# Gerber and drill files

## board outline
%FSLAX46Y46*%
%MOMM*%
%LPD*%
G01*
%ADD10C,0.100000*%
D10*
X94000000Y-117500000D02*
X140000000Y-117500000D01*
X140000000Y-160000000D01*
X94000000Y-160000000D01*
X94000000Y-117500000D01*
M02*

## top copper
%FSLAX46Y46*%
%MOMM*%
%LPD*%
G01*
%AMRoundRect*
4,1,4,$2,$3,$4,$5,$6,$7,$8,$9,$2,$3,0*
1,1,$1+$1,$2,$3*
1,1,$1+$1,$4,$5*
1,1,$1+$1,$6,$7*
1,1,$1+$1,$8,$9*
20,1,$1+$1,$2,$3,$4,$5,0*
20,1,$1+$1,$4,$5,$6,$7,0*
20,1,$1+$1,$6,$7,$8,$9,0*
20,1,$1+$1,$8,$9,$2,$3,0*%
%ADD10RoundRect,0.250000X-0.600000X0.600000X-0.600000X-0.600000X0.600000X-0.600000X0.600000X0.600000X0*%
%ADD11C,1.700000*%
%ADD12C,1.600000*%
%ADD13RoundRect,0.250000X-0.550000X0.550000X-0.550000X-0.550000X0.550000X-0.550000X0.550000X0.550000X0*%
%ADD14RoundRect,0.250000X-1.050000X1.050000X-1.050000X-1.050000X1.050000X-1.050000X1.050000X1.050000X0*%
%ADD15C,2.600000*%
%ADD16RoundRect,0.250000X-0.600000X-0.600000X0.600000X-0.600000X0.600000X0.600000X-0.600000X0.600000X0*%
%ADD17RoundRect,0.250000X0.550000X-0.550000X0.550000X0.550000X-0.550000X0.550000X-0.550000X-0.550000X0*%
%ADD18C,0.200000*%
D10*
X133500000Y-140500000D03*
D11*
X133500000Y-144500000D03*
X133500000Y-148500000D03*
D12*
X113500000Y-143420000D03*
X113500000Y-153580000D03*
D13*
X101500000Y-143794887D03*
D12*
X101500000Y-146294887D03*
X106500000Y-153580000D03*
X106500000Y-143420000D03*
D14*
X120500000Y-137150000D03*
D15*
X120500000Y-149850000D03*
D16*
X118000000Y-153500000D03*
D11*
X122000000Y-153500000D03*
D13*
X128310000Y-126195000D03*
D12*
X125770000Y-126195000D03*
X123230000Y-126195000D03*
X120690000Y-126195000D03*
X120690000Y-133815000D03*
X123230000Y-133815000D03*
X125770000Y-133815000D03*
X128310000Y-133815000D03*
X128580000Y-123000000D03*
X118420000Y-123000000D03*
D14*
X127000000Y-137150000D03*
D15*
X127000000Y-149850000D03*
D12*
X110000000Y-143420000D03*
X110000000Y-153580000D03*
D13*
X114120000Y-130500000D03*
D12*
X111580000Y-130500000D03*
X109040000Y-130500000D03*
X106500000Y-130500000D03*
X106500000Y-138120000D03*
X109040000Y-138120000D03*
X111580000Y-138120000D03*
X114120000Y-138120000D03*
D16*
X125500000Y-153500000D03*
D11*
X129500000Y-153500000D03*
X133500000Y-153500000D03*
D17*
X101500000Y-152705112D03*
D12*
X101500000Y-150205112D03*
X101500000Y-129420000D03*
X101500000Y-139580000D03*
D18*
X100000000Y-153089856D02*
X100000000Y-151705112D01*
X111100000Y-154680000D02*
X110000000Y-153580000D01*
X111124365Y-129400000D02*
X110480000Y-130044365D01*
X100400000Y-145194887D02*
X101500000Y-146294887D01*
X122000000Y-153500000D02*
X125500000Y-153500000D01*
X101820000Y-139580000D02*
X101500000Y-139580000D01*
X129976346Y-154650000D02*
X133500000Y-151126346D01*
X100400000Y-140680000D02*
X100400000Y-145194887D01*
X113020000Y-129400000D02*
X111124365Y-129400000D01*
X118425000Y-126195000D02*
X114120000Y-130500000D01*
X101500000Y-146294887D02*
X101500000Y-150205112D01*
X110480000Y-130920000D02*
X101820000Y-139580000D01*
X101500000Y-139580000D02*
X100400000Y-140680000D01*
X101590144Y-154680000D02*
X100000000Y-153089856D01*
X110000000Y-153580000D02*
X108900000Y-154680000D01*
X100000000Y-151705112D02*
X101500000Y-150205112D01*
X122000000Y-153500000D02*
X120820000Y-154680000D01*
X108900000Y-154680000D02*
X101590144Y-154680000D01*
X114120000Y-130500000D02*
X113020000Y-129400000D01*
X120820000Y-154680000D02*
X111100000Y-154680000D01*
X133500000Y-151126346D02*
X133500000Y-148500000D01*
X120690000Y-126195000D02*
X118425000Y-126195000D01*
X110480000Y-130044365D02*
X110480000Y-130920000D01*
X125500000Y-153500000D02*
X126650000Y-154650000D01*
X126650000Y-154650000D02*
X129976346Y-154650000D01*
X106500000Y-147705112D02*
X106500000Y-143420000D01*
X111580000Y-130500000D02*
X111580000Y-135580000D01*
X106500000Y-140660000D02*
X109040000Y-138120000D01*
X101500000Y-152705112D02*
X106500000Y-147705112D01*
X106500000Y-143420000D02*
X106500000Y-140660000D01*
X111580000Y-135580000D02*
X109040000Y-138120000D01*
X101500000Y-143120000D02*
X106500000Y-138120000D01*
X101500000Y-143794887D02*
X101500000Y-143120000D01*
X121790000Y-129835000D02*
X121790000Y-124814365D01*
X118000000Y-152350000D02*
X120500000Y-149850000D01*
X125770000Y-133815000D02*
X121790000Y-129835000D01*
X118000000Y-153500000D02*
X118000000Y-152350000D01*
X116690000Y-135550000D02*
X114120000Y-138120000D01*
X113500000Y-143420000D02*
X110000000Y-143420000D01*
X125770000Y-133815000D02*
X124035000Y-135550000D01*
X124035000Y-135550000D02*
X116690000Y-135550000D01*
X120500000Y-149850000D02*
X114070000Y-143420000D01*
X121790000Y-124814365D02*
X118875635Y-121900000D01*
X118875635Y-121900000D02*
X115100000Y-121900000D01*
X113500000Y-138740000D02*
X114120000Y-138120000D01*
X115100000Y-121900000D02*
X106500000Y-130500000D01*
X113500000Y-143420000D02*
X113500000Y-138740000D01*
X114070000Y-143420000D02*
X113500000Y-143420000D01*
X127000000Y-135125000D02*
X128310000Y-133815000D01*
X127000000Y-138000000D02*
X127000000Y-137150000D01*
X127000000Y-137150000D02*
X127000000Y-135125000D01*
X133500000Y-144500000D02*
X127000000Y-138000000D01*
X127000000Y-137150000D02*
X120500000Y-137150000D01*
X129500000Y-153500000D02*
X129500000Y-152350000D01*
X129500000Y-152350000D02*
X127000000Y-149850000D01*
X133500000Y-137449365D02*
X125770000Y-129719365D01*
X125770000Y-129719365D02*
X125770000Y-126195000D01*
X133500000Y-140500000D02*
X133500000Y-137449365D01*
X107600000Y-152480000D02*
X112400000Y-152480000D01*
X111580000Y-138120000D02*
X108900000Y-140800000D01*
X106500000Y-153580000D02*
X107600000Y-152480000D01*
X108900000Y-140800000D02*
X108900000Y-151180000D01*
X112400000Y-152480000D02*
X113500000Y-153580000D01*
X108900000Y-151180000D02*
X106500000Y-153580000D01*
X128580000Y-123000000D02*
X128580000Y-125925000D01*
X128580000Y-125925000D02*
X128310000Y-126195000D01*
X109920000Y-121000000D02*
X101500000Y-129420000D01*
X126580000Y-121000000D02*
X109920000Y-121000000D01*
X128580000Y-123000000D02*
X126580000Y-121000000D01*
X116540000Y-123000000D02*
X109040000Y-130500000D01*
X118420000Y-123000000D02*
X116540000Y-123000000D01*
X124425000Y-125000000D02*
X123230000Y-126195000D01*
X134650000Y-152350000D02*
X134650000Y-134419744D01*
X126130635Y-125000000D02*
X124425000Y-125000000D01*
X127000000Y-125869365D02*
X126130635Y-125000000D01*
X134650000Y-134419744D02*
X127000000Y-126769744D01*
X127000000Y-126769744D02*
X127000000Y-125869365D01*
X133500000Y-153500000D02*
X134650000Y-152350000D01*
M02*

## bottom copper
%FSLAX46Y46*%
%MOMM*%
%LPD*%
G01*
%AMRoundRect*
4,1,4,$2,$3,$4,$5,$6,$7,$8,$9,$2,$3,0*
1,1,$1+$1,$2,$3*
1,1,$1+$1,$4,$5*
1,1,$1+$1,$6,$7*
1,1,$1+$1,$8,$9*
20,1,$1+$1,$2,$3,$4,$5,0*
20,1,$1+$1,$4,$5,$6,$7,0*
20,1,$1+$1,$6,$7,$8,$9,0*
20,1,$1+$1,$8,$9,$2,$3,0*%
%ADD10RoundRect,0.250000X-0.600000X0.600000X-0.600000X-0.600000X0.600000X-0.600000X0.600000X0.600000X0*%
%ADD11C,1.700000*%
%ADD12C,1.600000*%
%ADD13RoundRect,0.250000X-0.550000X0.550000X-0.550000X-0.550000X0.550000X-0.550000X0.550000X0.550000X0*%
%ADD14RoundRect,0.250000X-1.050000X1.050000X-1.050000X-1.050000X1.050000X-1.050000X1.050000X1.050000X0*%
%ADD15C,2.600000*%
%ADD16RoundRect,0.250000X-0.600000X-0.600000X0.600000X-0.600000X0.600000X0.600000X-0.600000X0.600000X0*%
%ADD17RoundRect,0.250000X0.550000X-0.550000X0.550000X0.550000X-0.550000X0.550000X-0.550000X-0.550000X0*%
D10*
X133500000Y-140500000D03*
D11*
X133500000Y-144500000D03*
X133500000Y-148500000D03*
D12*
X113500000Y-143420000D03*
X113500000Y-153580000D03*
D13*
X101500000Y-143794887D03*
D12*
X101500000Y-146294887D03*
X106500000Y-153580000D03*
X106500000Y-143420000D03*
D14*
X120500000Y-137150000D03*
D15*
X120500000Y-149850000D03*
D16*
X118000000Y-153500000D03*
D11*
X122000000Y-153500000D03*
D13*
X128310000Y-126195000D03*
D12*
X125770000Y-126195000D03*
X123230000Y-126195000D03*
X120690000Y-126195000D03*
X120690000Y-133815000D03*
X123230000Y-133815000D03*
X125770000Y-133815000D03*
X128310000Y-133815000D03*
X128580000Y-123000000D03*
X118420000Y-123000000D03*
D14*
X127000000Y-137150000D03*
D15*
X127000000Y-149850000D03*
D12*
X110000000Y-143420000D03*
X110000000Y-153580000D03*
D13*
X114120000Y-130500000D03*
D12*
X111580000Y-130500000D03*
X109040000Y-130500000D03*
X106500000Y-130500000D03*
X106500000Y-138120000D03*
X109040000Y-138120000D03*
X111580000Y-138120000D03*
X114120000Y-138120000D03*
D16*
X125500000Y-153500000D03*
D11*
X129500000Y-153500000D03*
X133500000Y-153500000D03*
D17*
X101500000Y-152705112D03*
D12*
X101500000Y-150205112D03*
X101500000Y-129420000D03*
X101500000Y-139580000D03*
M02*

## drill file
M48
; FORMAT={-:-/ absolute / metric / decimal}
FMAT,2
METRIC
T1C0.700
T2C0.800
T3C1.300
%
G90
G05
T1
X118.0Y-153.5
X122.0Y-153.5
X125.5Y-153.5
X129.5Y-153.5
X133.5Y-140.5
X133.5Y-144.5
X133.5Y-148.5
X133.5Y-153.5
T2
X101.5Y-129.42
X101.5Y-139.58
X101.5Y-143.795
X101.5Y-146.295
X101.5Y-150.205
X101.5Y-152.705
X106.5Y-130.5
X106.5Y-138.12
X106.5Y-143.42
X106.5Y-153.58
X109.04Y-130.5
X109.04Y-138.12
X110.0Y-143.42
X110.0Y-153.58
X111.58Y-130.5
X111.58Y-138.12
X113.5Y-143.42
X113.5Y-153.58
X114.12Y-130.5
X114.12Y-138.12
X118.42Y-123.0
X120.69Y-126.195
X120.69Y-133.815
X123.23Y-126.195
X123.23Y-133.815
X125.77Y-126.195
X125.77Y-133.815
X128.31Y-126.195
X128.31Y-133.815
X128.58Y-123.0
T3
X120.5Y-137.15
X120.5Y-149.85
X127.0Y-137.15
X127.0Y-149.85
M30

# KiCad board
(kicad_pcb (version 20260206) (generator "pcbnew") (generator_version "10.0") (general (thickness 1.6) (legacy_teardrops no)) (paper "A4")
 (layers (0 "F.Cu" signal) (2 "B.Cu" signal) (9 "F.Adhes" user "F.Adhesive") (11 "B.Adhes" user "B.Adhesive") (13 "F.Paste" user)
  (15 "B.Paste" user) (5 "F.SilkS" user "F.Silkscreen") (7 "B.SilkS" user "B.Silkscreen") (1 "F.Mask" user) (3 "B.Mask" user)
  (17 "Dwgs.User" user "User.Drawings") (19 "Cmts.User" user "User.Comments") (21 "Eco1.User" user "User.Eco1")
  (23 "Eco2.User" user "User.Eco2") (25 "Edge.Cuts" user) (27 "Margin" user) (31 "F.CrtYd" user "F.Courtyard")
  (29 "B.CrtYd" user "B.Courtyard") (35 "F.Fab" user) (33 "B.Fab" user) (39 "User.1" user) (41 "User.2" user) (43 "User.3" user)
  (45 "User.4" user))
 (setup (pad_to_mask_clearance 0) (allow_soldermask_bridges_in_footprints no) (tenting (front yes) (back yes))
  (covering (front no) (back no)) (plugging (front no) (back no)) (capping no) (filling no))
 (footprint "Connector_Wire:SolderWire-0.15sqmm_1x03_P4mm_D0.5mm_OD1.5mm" (layer "F.Cu") (at 133.5 140.5 -90)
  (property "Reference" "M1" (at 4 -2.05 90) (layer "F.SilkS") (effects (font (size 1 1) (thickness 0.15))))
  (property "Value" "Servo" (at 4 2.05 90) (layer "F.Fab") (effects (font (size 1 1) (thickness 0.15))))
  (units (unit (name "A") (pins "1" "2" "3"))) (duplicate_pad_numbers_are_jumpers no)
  (pad "1" thru_hole roundrect (at 0 0 270) (size 1.7 1.7) (drill 0.7) (layers "*.Cu" "*.Mask") (remove_unused_layers no)
   (roundrect_rratio 0.147059) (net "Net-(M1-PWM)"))
  (pad "2" thru_hole circle (at 4 0 270) (size 1.7 1.7) (drill 0.7) (layers "*.Cu" "*.Mask") (remove_unused_layers no) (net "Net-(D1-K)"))
  (pad "3" thru_hole circle (at 8 0 270) (size 1.7 1.7) (drill 0.7) (layers "*.Cu" "*.Mask") (remove_unused_layers no) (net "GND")))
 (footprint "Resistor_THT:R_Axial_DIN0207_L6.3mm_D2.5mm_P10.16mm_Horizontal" (layer "F.Cu") (at 113.5 143.42 -90)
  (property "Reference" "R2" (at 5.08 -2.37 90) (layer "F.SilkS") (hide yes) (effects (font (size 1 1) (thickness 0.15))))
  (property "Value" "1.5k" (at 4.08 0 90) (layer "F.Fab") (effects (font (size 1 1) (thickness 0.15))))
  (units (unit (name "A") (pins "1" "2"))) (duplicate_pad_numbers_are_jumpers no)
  (pad "1" thru_hole circle (at 0 0 270) (size 1.6 1.6) (drill 0.8) (layers "*.Cu" "*.Mask") (remove_unused_layers no) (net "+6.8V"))
  (pad "2" thru_hole circle (at 10.16 0 270) (size 1.6 1.6) (drill 0.8) (layers "*.Cu" "*.Mask") (remove_unused_layers no)
   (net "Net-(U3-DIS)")))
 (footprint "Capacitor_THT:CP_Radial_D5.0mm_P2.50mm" (layer "F.Cu") (at 101.5 143.794887 -90)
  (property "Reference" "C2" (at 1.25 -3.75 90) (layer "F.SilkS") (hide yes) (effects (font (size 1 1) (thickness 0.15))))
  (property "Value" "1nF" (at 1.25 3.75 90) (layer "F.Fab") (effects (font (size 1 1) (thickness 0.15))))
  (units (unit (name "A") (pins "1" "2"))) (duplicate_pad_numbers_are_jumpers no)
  (pad "1" thru_hole roundrect (at 0 0 270) (size 1.6 1.6) (drill 0.8) (layers "*.Cu" "*.Mask") (remove_unused_layers no)
   (roundrect_rratio 0.15625) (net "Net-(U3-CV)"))
  (pad "2" thru_hole circle (at 2.5 0 270) (size 1.6 1.6) (drill 0.8) (layers "*.Cu" "*.Mask") (remove_unused_layers no) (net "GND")))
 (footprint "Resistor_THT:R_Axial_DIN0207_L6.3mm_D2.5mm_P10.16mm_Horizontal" (layer "F.Cu") (at 106.5 153.58 90)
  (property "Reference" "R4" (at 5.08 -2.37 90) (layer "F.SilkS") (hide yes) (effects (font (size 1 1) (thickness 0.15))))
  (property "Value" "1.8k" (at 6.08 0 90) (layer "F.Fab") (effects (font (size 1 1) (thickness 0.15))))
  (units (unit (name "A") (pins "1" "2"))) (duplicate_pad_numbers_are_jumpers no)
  (pad "1" thru_hole circle (at 0 0 90) (size 1.6 1.6) (drill 0.8) (layers "*.Cu" "*.Mask") (remove_unused_layers no) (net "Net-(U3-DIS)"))
  (pad "2" thru_hole circle (at 10.16 0 90) (size 1.6 1.6) (drill 0.8) (layers "*.Cu" "*.Mask") (remove_unused_layers no)
   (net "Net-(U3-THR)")))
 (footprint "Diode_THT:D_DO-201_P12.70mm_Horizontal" (layer "F.Cu") (at 120.5 137.15 -90)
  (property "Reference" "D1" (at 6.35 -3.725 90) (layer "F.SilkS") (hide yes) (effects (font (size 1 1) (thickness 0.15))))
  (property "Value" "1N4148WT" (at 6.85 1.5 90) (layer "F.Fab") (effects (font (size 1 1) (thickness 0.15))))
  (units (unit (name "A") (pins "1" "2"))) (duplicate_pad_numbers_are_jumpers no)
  (pad "1" thru_hole roundrect (at 0 0 270) (size 2.6 2.6) (drill 1.3) (layers "*.Cu" "*.Mask") (remove_unused_layers no)
   (roundrect_rratio 0.096154) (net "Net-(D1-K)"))
  (pad "2" thru_hole circle (at 12.7 0 270) (size 2.6 2.6) (drill 1.3) (layers "*.Cu" "*.Mask") (remove_unused_layers no) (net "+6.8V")))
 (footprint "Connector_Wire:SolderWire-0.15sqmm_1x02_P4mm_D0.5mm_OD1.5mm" (layer "F.Cu") (at 118 153.5)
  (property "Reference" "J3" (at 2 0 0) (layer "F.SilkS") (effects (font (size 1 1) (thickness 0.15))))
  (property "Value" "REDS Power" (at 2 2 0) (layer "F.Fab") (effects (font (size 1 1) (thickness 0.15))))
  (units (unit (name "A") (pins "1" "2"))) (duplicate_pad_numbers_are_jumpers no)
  (pad "1" thru_hole roundrect (at 0 0) (size 1.7 1.7) (drill 0.7) (layers "*.Cu" "*.Mask") (remove_unused_layers no)
   (roundrect_rratio 0.147059) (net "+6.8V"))
  (pad "2" thru_hole circle (at 4 0) (size 1.7 1.7) (drill 0.7) (layers "*.Cu" "*.Mask") (remove_unused_layers no) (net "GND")))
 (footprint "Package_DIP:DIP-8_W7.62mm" (layer "F.Cu") (at 128.31 126.195 -90)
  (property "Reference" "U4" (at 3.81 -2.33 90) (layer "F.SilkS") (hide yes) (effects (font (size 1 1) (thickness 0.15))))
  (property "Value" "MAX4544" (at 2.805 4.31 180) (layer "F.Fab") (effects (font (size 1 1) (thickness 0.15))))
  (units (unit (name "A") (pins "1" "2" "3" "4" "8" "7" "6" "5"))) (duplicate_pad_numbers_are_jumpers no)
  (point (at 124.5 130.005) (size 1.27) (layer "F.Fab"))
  (pad "1" thru_hole roundrect (at 0 0 270) (size 1.6 1.6) (drill 0.8) (layers "*.Cu" "*.Mask") (remove_unused_layers no)
   (roundrect_rratio 0.15625) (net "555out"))
  (pad "2" thru_hole circle (at 0 2.54 270) (size 1.6 1.6) (drill 0.8) (layers "*.Cu" "*.Mask") (remove_unused_layers no)
   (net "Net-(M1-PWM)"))
  (pad "3" thru_hole circle (at 0 5.08 270) (size 1.6 1.6) (drill 0.8) (layers "*.Cu" "*.Mask") (remove_unused_layers no) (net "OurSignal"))
  (pad "4" thru_hole circle (at 0 7.62 270) (size 1.6 1.6) (drill 0.8) (layers "*.Cu" "*.Mask") (remove_unused_layers no) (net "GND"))
  (pad "5" thru_hole circle (at 7.62 7.62 270) (size 1.6 1.6) (drill 0.8) (layers "*.Cu" "*.Mask") (remove_unused_layers no)
   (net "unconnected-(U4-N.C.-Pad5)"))
  (pad "6" thru_hole circle (at 7.62 5.08 270) (size 1.6 1.6) (drill 0.8) (layers "*.Cu" "*.Mask") (remove_unused_layers no)
   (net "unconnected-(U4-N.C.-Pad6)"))
  (pad "7" thru_hole circle (at 7.62 2.54 270) (size 1.6 1.6) (drill 0.8) (layers "*.Cu" "*.Mask") (remove_unused_layers no) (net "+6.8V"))
  (pad "8" thru_hole circle (at 7.62 0 270) (size 1.6 1.6) (drill 0.8) (layers "*.Cu" "*.Mask") (remove_unused_layers no) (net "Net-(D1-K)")))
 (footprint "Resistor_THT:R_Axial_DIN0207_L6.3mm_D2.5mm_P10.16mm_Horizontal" (layer "F.Cu") (at 128.58 123 180)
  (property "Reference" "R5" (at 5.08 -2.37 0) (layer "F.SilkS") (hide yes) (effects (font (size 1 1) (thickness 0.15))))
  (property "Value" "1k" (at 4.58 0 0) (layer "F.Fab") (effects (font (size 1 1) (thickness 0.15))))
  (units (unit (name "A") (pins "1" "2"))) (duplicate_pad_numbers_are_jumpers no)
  (pad "1" thru_hole circle (at 0 0 180) (size 1.6 1.6) (drill 0.8) (layers "*.Cu" "*.Mask") (remove_unused_layers no) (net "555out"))
  (pad "2" thru_hole circle (at 10.16 0 180) (size 1.6 1.6) (drill 0.8) (layers "*.Cu" "*.Mask") (remove_unused_layers no)
   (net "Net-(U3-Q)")))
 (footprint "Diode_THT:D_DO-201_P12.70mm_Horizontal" (layer "F.Cu") (at 127 137.15 -90)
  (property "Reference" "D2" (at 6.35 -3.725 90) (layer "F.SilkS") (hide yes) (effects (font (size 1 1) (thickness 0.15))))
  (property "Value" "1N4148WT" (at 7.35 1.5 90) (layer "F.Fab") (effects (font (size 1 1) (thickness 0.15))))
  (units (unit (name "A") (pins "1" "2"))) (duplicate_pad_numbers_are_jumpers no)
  (pad "1" thru_hole roundrect (at 0 0 270) (size 2.6 2.6) (drill 1.3) (layers "*.Cu" "*.Mask") (remove_unused_layers no)
   (roundrect_rratio 0.096154) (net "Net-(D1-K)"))
  (pad "2" thru_hole circle (at 12.7 0 270) (size 2.6 2.6) (drill 1.3) (layers "*.Cu" "*.Mask") (remove_unused_layers no) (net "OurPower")))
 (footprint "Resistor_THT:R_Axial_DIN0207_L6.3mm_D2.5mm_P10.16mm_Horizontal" (layer "F.Cu") (at 110 143.42 -90)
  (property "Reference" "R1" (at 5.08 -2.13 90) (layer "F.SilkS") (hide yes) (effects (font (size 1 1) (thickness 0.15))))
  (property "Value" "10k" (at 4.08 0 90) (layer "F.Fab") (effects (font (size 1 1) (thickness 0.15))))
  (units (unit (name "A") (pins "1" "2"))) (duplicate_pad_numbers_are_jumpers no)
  (pad "1" thru_hole circle (at 0 0 270) (size 1.6 1.6) (drill 0.8) (layers "*.Cu" "*.Mask") (remove_unused_layers no) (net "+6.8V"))
  (pad "2" thru_hole circle (at 10.16 0 270) (size 1.6 1.6) (drill 0.8) (layers "*.Cu" "*.Mask") (remove_unused_layers no) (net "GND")))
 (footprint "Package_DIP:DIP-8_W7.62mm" (layer "F.Cu") (at 114.12 130.5 -90)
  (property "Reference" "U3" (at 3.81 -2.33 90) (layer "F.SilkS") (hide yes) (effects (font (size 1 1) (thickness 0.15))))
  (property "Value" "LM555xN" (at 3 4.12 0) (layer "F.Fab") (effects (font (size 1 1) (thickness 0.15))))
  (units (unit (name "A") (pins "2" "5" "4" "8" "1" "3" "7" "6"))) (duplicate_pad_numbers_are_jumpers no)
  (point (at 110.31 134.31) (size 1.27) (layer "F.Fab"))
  (pad "1" thru_hole roundrect (at 0 0 270) (size 1.6 1.6) (drill 0.8) (layers "*.Cu" "*.Mask") (remove_unused_layers no)
   (roundrect_rratio 0.15625) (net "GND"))
  (pad "2" thru_hole circle (at 0 2.54 270) (size 1.6 1.6) (drill 0.8) (layers "*.Cu" "*.Mask") (remove_unused_layers no)
   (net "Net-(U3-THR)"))
  (pad "3" thru_hole circle (at 0 5.08 270) (size 1.6 1.6) (drill 0.8) (layers "*.Cu" "*.Mask") (remove_unused_layers no) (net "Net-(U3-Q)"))
  (pad "4" thru_hole circle (at 0 7.62 270) (size 1.6 1.6) (drill 0.8) (layers "*.Cu" "*.Mask") (remove_unused_layers no) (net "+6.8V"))
  (pad "5" thru_hole circle (at 7.62 7.62 270) (size 1.6 1.6) (drill 0.8) (layers "*.Cu" "*.Mask") (remove_unused_layers no)
   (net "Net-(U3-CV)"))
  (pad "6" thru_hole circle (at 7.62 5.08 270) (size 1.6 1.6) (drill 0.8) (layers "*.Cu" "*.Mask") (remove_unused_layers no)
   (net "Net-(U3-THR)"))
  (pad "7" thru_hole circle (at 7.62 2.54 270) (size 1.6 1.6) (drill 0.8) (layers "*.Cu" "*.Mask") (remove_unused_layers no)
   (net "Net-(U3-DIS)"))
  (pad "8" thru_hole circle (at 7.62 0 270) (size 1.6 1.6) (drill 0.8) (layers "*.Cu" "*.Mask") (remove_unused_layers no) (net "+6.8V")))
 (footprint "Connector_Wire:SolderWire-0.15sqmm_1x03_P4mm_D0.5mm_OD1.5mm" (layer "F.Cu") (at 125.5 153.5)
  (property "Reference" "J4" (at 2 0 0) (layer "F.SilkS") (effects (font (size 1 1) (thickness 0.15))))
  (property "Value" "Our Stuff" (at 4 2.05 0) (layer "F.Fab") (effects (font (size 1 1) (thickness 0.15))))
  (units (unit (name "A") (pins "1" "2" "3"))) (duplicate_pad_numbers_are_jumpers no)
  (pad "1" thru_hole roundrect (at 0 0) (size 1.7 1.7) (drill 0.7) (layers "*.Cu" "*.Mask") (remove_unused_layers no)
   (roundrect_rratio 0.147059) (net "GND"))
  (pad "2" thru_hole circle (at 4 0) (size 1.7 1.7) (drill 0.7) (layers "*.Cu" "*.Mask") (remove_unused_layers no) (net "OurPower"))
  (pad "3" thru_hole circle (at 8 0) (size 1.7 1.7) (drill 0.7) (layers "*.Cu" "*.Mask") (remove_unused_layers no) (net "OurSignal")))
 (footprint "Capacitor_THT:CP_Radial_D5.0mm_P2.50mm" (layer "F.Cu") (at 101.5 152.705112 90)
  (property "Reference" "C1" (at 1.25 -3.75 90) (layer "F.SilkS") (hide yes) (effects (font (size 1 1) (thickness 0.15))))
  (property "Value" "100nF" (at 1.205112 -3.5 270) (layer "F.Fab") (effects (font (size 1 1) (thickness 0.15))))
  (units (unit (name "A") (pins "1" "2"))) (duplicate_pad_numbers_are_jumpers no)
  (pad "1" thru_hole roundrect (at 0 0 90) (size 1.6 1.6) (drill 0.8) (layers "*.Cu" "*.Mask") (remove_unused_layers no)
   (roundrect_rratio 0.15625) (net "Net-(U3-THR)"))
  (pad "2" thru_hole circle (at 2.5 0 90) (size 1.6 1.6) (drill 0.8) (layers "*.Cu" "*.Mask") (remove_unused_layers no) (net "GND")))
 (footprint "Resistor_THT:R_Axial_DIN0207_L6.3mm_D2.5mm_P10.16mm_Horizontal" (layer "F.Cu") (at 101.5 129.42 -90)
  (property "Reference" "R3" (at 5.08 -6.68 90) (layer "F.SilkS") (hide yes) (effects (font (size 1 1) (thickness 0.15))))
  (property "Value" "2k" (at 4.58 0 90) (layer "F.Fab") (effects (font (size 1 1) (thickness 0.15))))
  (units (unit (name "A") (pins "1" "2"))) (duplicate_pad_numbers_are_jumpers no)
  (pad "1" thru_hole circle (at 0 0 270) (size 1.6 1.6) (drill 0.8) (layers "*.Cu" "*.Mask") (remove_unused_layers no) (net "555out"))
  (pad "2" thru_hole circle (at 10.16 0 270) (size 1.6 1.6) (drill 0.8) (layers "*.Cu" "*.Mask") (remove_unused_layers no) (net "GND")))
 (gr_rect (start 94 117.5) (end 140 160) (stroke (width 0.1) (type default)) (fill no) (layer "Edge.Cuts"))
 (segment (start 100 153.089856) (end 100 151.705112) (width 0.2) (layer "F.Cu") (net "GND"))
 (segment (start 111.1 154.68) (end 110 153.58) (width 0.2) (layer "F.Cu") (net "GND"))
 (segment (start 111.124365 129.4) (end 110.48 130.044365) (width 0.2) (layer "F.Cu") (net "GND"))
 (segment (start 100.4 145.194887) (end 101.5 146.294887) (width 0.2) (layer "F.Cu") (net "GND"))
 (segment (start 122 153.5) (end 125.5 153.5) (width 0.2) (layer "F.Cu") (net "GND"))
 (segment (start 101.82 139.58) (end 101.5 139.58) (width 0.2) (layer "F.Cu") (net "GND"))
 (segment (start 129.976346 154.65) (end 133.5 151.126346) (width 0.2) (layer "F.Cu") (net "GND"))
 (segment (start 100.4 140.68) (end 100.4 145.194887) (width 0.2) (layer "F.Cu") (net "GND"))
 (segment (start 113.02 129.4) (end 111.124365 129.4) (width 0.2) (layer "F.Cu") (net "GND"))
 (segment (start 118.425 126.195) (end 114.12 130.5) (width 0.2) (layer "F.Cu") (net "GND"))
 (segment (start 101.5 146.294887) (end 101.5 150.205112) (width 0.2) (layer "F.Cu") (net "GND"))
 (segment (start 110.48 130.92) (end 101.82 139.58) (width 0.2) (layer "F.Cu") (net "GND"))
 (segment (start 101.5 139.58) (end 100.4 140.68) (width 0.2) (layer "F.Cu") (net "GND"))
 (segment (start 101.590144 154.68) (end 100 153.089856) (width 0.2) (layer "F.Cu") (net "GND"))
 (segment (start 110 153.58) (end 108.9 154.68) (width 0.2) (layer "F.Cu") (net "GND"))
 (segment (start 100 151.705112) (end 101.5 150.205112) (width 0.2) (layer "F.Cu") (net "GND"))
 (segment (start 122 153.5) (end 120.82 154.68) (width 0.2) (layer "F.Cu") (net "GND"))
 (segment (start 108.9 154.68) (end 101.590144 154.68) (width 0.2) (layer "F.Cu") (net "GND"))
 (segment (start 114.12 130.5) (end 113.02 129.4) (width 0.2) (layer "F.Cu") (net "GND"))
 (segment (start 120.82 154.68) (end 111.1 154.68) (width 0.2) (layer "F.Cu") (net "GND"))
 (segment (start 133.5 151.126346) (end 133.5 148.5) (width 0.2) (layer "F.Cu") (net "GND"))
 (segment (start 120.69 126.195) (end 118.425 126.195) (width 0.2) (layer "F.Cu") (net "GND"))
 (segment (start 110.48 130.044365) (end 110.48 130.92) (width 0.2) (layer "F.Cu") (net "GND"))
 (segment (start 125.5 153.5) (end 126.65 154.65) (width 0.2) (layer "F.Cu") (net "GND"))
 (segment (start 126.65 154.65) (end 129.976346 154.65) (width 0.2) (layer "F.Cu") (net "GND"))
 (segment (start 106.5 147.705112) (end 106.5 143.42) (width 0.2) (layer "F.Cu") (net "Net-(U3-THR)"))
 (segment (start 111.58 130.5) (end 111.58 135.58) (width 0.2) (layer "F.Cu") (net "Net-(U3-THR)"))
 (segment (start 106.5 140.66) (end 109.04 138.12) (width 0.2) (layer "F.Cu") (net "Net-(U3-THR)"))
 (segment (start 101.5 152.705112) (end 106.5 147.705112) (width 0.2) (layer "F.Cu") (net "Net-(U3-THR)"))
 (segment (start 106.5 143.42) (end 106.5 140.66) (width 0.2) (layer "F.Cu") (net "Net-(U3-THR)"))
 (segment (start 111.58 135.58) (end 109.04 138.12) (width 0.2) (layer "F.Cu") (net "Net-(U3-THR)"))
 (segment (start 101.5 143.12) (end 106.5 138.12) (width 0.2) (layer "F.Cu") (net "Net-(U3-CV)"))
 (segment (start 101.5 143.794887) (end 101.5 143.12) (width 0.2) (layer "F.Cu") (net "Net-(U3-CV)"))
 (segment (start 121.79 129.835) (end 121.79 124.814365) (width 0.2) (layer "F.Cu") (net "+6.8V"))
 (segment (start 118 152.35) (end 120.5 149.85) (width 0.2) (layer "F.Cu") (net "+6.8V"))
 (segment (start 125.77 133.815) (end 121.79 129.835) (width 0.2) (layer "F.Cu") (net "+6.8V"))
 (segment (start 118 153.5) (end 118 152.35) (width 0.2) (layer "F.Cu") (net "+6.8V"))
 (segment (start 116.69 135.55) (end 114.12 138.12) (width 0.2) (layer "F.Cu") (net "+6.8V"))
 (segment (start 113.5 143.42) (end 110 143.42) (width 0.2) (layer "F.Cu") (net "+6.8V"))
 (segment (start 125.77 133.815) (end 124.035 135.55) (width 0.2) (layer "F.Cu") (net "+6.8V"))
 (segment (start 124.035 135.55) (end 116.69 135.55) (width 0.2) (layer "F.Cu") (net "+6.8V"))
 (segment (start 120.5 149.85) (end 114.07 143.42) (width 0.2) (layer "F.Cu") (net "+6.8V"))
 (segment (start 121.79 124.814365) (end 118.875635 121.9) (width 0.2) (layer "F.Cu") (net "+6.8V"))
 (segment (start 118.875635 121.9) (end 115.1 121.9) (width 0.2) (layer "F.Cu") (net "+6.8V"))
 (segment (start 113.5 138.74) (end 114.12 138.12) (width 0.2) (layer "F.Cu") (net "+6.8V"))
 (segment (start 115.1 121.9) (end 106.5 130.5) (width 0.2) (layer "F.Cu") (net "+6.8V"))
 (segment (start 113.5 143.42) (end 113.5 138.74) (width 0.2) (layer "F.Cu") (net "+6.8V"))
 (segment (start 114.07 143.42) (end 113.5 143.42) (width 0.2) (layer "F.Cu") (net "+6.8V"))
 (segment (start 127 135.125) (end 128.31 133.815) (width 0.2) (layer "F.Cu") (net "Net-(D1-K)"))
 (segment (start 127 138) (end 127 137.15) (width 0.2) (layer "F.Cu") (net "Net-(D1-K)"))
 (segment (start 127 137.15) (end 127 135.125) (width 0.2) (layer "F.Cu") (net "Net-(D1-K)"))
 (segment (start 133.5 144.5) (end 127 138) (width 0.2) (layer "F.Cu") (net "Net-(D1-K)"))
 (segment (start 127 137.15) (end 120.5 137.15) (width 0.2) (layer "F.Cu") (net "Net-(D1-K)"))
 (segment (start 129.5 153.5) (end 129.5 152.35) (width 0.2) (layer "F.Cu") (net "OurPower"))
 (segment (start 129.5 152.35) (end 127 149.85) (width 0.2) (layer "F.Cu") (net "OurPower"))
 (segment (start 133.5 137.449365) (end 125.77 129.719365) (width 0.2) (layer "F.Cu") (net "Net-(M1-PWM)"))
 (segment (start 125.77 129.719365) (end 125.77 126.195) (width 0.2) (layer "F.Cu") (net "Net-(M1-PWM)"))
 (segment (start 133.5 140.5) (end 133.5 137.449365) (width 0.2) (layer "F.Cu") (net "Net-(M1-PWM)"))
 (segment (start 107.6 152.48) (end 112.4 152.48) (width 0.2) (layer "F.Cu") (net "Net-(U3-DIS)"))
 (segment (start 111.58 138.12) (end 108.9 140.8) (width 0.2) (layer "F.Cu") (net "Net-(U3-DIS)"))
 (segment (start 106.5 153.58) (end 107.6 152.48) (width 0.2) (layer "F.Cu") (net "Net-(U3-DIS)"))
 (segment (start 108.9 140.8) (end 108.9 151.18) (width 0.2) (layer "F.Cu") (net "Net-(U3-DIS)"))
 (segment (start 112.4 152.48) (end 113.5 153.58) (width 0.2) (layer "F.Cu") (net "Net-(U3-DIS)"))
 (segment (start 108.9 151.18) (end 106.5 153.58) (width 0.2) (layer "F.Cu") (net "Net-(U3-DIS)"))
 (segment (start 128.58 123) (end 128.58 125.925) (width 0.2) (layer "F.Cu") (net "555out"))
 (segment (start 128.58 125.925) (end 128.31 126.195) (width 0.2) (layer "F.Cu") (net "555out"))
 (segment (start 109.92 121) (end 101.5 129.42) (width 0.2) (layer "F.Cu") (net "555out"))
 (segment (start 126.58 121) (end 109.92 121) (width 0.2) (layer "F.Cu") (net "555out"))
 (segment (start 128.58 123) (end 126.58 121) (width 0.2) (layer "F.Cu") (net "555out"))
 (segment (start 116.54 123) (end 109.04 130.5) (width 0.2) (layer "F.Cu") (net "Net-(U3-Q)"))
 (segment (start 118.42 123) (end 116.54 123) (width 0.2) (layer "F.Cu") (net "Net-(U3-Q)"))
 (segment (start 124.425 125) (end 123.23 126.195) (width 0.2) (layer "F.Cu") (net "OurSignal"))
 (segment (start 134.65 152.35) (end 134.65 134.419744) (width 0.2) (layer "F.Cu") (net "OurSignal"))
 (segment (start 126.130635 125) (end 124.425 125) (width 0.2) (layer "F.Cu") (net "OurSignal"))
 (segment (start 127 125.869365) (end 126.130635 125) (width 0.2) (layer "F.Cu") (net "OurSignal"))
 (segment (start 134.65 134.419744) (end 127 126.769744) (width 0.2) (layer "F.Cu") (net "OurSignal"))
 (segment (start 127 126.769744) (end 127 125.869365) (width 0.2) (layer "F.Cu") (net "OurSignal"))
 (segment (start 133.5 153.5) (end 134.65 152.35) (width 0.2) (layer "F.Cu") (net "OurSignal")))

